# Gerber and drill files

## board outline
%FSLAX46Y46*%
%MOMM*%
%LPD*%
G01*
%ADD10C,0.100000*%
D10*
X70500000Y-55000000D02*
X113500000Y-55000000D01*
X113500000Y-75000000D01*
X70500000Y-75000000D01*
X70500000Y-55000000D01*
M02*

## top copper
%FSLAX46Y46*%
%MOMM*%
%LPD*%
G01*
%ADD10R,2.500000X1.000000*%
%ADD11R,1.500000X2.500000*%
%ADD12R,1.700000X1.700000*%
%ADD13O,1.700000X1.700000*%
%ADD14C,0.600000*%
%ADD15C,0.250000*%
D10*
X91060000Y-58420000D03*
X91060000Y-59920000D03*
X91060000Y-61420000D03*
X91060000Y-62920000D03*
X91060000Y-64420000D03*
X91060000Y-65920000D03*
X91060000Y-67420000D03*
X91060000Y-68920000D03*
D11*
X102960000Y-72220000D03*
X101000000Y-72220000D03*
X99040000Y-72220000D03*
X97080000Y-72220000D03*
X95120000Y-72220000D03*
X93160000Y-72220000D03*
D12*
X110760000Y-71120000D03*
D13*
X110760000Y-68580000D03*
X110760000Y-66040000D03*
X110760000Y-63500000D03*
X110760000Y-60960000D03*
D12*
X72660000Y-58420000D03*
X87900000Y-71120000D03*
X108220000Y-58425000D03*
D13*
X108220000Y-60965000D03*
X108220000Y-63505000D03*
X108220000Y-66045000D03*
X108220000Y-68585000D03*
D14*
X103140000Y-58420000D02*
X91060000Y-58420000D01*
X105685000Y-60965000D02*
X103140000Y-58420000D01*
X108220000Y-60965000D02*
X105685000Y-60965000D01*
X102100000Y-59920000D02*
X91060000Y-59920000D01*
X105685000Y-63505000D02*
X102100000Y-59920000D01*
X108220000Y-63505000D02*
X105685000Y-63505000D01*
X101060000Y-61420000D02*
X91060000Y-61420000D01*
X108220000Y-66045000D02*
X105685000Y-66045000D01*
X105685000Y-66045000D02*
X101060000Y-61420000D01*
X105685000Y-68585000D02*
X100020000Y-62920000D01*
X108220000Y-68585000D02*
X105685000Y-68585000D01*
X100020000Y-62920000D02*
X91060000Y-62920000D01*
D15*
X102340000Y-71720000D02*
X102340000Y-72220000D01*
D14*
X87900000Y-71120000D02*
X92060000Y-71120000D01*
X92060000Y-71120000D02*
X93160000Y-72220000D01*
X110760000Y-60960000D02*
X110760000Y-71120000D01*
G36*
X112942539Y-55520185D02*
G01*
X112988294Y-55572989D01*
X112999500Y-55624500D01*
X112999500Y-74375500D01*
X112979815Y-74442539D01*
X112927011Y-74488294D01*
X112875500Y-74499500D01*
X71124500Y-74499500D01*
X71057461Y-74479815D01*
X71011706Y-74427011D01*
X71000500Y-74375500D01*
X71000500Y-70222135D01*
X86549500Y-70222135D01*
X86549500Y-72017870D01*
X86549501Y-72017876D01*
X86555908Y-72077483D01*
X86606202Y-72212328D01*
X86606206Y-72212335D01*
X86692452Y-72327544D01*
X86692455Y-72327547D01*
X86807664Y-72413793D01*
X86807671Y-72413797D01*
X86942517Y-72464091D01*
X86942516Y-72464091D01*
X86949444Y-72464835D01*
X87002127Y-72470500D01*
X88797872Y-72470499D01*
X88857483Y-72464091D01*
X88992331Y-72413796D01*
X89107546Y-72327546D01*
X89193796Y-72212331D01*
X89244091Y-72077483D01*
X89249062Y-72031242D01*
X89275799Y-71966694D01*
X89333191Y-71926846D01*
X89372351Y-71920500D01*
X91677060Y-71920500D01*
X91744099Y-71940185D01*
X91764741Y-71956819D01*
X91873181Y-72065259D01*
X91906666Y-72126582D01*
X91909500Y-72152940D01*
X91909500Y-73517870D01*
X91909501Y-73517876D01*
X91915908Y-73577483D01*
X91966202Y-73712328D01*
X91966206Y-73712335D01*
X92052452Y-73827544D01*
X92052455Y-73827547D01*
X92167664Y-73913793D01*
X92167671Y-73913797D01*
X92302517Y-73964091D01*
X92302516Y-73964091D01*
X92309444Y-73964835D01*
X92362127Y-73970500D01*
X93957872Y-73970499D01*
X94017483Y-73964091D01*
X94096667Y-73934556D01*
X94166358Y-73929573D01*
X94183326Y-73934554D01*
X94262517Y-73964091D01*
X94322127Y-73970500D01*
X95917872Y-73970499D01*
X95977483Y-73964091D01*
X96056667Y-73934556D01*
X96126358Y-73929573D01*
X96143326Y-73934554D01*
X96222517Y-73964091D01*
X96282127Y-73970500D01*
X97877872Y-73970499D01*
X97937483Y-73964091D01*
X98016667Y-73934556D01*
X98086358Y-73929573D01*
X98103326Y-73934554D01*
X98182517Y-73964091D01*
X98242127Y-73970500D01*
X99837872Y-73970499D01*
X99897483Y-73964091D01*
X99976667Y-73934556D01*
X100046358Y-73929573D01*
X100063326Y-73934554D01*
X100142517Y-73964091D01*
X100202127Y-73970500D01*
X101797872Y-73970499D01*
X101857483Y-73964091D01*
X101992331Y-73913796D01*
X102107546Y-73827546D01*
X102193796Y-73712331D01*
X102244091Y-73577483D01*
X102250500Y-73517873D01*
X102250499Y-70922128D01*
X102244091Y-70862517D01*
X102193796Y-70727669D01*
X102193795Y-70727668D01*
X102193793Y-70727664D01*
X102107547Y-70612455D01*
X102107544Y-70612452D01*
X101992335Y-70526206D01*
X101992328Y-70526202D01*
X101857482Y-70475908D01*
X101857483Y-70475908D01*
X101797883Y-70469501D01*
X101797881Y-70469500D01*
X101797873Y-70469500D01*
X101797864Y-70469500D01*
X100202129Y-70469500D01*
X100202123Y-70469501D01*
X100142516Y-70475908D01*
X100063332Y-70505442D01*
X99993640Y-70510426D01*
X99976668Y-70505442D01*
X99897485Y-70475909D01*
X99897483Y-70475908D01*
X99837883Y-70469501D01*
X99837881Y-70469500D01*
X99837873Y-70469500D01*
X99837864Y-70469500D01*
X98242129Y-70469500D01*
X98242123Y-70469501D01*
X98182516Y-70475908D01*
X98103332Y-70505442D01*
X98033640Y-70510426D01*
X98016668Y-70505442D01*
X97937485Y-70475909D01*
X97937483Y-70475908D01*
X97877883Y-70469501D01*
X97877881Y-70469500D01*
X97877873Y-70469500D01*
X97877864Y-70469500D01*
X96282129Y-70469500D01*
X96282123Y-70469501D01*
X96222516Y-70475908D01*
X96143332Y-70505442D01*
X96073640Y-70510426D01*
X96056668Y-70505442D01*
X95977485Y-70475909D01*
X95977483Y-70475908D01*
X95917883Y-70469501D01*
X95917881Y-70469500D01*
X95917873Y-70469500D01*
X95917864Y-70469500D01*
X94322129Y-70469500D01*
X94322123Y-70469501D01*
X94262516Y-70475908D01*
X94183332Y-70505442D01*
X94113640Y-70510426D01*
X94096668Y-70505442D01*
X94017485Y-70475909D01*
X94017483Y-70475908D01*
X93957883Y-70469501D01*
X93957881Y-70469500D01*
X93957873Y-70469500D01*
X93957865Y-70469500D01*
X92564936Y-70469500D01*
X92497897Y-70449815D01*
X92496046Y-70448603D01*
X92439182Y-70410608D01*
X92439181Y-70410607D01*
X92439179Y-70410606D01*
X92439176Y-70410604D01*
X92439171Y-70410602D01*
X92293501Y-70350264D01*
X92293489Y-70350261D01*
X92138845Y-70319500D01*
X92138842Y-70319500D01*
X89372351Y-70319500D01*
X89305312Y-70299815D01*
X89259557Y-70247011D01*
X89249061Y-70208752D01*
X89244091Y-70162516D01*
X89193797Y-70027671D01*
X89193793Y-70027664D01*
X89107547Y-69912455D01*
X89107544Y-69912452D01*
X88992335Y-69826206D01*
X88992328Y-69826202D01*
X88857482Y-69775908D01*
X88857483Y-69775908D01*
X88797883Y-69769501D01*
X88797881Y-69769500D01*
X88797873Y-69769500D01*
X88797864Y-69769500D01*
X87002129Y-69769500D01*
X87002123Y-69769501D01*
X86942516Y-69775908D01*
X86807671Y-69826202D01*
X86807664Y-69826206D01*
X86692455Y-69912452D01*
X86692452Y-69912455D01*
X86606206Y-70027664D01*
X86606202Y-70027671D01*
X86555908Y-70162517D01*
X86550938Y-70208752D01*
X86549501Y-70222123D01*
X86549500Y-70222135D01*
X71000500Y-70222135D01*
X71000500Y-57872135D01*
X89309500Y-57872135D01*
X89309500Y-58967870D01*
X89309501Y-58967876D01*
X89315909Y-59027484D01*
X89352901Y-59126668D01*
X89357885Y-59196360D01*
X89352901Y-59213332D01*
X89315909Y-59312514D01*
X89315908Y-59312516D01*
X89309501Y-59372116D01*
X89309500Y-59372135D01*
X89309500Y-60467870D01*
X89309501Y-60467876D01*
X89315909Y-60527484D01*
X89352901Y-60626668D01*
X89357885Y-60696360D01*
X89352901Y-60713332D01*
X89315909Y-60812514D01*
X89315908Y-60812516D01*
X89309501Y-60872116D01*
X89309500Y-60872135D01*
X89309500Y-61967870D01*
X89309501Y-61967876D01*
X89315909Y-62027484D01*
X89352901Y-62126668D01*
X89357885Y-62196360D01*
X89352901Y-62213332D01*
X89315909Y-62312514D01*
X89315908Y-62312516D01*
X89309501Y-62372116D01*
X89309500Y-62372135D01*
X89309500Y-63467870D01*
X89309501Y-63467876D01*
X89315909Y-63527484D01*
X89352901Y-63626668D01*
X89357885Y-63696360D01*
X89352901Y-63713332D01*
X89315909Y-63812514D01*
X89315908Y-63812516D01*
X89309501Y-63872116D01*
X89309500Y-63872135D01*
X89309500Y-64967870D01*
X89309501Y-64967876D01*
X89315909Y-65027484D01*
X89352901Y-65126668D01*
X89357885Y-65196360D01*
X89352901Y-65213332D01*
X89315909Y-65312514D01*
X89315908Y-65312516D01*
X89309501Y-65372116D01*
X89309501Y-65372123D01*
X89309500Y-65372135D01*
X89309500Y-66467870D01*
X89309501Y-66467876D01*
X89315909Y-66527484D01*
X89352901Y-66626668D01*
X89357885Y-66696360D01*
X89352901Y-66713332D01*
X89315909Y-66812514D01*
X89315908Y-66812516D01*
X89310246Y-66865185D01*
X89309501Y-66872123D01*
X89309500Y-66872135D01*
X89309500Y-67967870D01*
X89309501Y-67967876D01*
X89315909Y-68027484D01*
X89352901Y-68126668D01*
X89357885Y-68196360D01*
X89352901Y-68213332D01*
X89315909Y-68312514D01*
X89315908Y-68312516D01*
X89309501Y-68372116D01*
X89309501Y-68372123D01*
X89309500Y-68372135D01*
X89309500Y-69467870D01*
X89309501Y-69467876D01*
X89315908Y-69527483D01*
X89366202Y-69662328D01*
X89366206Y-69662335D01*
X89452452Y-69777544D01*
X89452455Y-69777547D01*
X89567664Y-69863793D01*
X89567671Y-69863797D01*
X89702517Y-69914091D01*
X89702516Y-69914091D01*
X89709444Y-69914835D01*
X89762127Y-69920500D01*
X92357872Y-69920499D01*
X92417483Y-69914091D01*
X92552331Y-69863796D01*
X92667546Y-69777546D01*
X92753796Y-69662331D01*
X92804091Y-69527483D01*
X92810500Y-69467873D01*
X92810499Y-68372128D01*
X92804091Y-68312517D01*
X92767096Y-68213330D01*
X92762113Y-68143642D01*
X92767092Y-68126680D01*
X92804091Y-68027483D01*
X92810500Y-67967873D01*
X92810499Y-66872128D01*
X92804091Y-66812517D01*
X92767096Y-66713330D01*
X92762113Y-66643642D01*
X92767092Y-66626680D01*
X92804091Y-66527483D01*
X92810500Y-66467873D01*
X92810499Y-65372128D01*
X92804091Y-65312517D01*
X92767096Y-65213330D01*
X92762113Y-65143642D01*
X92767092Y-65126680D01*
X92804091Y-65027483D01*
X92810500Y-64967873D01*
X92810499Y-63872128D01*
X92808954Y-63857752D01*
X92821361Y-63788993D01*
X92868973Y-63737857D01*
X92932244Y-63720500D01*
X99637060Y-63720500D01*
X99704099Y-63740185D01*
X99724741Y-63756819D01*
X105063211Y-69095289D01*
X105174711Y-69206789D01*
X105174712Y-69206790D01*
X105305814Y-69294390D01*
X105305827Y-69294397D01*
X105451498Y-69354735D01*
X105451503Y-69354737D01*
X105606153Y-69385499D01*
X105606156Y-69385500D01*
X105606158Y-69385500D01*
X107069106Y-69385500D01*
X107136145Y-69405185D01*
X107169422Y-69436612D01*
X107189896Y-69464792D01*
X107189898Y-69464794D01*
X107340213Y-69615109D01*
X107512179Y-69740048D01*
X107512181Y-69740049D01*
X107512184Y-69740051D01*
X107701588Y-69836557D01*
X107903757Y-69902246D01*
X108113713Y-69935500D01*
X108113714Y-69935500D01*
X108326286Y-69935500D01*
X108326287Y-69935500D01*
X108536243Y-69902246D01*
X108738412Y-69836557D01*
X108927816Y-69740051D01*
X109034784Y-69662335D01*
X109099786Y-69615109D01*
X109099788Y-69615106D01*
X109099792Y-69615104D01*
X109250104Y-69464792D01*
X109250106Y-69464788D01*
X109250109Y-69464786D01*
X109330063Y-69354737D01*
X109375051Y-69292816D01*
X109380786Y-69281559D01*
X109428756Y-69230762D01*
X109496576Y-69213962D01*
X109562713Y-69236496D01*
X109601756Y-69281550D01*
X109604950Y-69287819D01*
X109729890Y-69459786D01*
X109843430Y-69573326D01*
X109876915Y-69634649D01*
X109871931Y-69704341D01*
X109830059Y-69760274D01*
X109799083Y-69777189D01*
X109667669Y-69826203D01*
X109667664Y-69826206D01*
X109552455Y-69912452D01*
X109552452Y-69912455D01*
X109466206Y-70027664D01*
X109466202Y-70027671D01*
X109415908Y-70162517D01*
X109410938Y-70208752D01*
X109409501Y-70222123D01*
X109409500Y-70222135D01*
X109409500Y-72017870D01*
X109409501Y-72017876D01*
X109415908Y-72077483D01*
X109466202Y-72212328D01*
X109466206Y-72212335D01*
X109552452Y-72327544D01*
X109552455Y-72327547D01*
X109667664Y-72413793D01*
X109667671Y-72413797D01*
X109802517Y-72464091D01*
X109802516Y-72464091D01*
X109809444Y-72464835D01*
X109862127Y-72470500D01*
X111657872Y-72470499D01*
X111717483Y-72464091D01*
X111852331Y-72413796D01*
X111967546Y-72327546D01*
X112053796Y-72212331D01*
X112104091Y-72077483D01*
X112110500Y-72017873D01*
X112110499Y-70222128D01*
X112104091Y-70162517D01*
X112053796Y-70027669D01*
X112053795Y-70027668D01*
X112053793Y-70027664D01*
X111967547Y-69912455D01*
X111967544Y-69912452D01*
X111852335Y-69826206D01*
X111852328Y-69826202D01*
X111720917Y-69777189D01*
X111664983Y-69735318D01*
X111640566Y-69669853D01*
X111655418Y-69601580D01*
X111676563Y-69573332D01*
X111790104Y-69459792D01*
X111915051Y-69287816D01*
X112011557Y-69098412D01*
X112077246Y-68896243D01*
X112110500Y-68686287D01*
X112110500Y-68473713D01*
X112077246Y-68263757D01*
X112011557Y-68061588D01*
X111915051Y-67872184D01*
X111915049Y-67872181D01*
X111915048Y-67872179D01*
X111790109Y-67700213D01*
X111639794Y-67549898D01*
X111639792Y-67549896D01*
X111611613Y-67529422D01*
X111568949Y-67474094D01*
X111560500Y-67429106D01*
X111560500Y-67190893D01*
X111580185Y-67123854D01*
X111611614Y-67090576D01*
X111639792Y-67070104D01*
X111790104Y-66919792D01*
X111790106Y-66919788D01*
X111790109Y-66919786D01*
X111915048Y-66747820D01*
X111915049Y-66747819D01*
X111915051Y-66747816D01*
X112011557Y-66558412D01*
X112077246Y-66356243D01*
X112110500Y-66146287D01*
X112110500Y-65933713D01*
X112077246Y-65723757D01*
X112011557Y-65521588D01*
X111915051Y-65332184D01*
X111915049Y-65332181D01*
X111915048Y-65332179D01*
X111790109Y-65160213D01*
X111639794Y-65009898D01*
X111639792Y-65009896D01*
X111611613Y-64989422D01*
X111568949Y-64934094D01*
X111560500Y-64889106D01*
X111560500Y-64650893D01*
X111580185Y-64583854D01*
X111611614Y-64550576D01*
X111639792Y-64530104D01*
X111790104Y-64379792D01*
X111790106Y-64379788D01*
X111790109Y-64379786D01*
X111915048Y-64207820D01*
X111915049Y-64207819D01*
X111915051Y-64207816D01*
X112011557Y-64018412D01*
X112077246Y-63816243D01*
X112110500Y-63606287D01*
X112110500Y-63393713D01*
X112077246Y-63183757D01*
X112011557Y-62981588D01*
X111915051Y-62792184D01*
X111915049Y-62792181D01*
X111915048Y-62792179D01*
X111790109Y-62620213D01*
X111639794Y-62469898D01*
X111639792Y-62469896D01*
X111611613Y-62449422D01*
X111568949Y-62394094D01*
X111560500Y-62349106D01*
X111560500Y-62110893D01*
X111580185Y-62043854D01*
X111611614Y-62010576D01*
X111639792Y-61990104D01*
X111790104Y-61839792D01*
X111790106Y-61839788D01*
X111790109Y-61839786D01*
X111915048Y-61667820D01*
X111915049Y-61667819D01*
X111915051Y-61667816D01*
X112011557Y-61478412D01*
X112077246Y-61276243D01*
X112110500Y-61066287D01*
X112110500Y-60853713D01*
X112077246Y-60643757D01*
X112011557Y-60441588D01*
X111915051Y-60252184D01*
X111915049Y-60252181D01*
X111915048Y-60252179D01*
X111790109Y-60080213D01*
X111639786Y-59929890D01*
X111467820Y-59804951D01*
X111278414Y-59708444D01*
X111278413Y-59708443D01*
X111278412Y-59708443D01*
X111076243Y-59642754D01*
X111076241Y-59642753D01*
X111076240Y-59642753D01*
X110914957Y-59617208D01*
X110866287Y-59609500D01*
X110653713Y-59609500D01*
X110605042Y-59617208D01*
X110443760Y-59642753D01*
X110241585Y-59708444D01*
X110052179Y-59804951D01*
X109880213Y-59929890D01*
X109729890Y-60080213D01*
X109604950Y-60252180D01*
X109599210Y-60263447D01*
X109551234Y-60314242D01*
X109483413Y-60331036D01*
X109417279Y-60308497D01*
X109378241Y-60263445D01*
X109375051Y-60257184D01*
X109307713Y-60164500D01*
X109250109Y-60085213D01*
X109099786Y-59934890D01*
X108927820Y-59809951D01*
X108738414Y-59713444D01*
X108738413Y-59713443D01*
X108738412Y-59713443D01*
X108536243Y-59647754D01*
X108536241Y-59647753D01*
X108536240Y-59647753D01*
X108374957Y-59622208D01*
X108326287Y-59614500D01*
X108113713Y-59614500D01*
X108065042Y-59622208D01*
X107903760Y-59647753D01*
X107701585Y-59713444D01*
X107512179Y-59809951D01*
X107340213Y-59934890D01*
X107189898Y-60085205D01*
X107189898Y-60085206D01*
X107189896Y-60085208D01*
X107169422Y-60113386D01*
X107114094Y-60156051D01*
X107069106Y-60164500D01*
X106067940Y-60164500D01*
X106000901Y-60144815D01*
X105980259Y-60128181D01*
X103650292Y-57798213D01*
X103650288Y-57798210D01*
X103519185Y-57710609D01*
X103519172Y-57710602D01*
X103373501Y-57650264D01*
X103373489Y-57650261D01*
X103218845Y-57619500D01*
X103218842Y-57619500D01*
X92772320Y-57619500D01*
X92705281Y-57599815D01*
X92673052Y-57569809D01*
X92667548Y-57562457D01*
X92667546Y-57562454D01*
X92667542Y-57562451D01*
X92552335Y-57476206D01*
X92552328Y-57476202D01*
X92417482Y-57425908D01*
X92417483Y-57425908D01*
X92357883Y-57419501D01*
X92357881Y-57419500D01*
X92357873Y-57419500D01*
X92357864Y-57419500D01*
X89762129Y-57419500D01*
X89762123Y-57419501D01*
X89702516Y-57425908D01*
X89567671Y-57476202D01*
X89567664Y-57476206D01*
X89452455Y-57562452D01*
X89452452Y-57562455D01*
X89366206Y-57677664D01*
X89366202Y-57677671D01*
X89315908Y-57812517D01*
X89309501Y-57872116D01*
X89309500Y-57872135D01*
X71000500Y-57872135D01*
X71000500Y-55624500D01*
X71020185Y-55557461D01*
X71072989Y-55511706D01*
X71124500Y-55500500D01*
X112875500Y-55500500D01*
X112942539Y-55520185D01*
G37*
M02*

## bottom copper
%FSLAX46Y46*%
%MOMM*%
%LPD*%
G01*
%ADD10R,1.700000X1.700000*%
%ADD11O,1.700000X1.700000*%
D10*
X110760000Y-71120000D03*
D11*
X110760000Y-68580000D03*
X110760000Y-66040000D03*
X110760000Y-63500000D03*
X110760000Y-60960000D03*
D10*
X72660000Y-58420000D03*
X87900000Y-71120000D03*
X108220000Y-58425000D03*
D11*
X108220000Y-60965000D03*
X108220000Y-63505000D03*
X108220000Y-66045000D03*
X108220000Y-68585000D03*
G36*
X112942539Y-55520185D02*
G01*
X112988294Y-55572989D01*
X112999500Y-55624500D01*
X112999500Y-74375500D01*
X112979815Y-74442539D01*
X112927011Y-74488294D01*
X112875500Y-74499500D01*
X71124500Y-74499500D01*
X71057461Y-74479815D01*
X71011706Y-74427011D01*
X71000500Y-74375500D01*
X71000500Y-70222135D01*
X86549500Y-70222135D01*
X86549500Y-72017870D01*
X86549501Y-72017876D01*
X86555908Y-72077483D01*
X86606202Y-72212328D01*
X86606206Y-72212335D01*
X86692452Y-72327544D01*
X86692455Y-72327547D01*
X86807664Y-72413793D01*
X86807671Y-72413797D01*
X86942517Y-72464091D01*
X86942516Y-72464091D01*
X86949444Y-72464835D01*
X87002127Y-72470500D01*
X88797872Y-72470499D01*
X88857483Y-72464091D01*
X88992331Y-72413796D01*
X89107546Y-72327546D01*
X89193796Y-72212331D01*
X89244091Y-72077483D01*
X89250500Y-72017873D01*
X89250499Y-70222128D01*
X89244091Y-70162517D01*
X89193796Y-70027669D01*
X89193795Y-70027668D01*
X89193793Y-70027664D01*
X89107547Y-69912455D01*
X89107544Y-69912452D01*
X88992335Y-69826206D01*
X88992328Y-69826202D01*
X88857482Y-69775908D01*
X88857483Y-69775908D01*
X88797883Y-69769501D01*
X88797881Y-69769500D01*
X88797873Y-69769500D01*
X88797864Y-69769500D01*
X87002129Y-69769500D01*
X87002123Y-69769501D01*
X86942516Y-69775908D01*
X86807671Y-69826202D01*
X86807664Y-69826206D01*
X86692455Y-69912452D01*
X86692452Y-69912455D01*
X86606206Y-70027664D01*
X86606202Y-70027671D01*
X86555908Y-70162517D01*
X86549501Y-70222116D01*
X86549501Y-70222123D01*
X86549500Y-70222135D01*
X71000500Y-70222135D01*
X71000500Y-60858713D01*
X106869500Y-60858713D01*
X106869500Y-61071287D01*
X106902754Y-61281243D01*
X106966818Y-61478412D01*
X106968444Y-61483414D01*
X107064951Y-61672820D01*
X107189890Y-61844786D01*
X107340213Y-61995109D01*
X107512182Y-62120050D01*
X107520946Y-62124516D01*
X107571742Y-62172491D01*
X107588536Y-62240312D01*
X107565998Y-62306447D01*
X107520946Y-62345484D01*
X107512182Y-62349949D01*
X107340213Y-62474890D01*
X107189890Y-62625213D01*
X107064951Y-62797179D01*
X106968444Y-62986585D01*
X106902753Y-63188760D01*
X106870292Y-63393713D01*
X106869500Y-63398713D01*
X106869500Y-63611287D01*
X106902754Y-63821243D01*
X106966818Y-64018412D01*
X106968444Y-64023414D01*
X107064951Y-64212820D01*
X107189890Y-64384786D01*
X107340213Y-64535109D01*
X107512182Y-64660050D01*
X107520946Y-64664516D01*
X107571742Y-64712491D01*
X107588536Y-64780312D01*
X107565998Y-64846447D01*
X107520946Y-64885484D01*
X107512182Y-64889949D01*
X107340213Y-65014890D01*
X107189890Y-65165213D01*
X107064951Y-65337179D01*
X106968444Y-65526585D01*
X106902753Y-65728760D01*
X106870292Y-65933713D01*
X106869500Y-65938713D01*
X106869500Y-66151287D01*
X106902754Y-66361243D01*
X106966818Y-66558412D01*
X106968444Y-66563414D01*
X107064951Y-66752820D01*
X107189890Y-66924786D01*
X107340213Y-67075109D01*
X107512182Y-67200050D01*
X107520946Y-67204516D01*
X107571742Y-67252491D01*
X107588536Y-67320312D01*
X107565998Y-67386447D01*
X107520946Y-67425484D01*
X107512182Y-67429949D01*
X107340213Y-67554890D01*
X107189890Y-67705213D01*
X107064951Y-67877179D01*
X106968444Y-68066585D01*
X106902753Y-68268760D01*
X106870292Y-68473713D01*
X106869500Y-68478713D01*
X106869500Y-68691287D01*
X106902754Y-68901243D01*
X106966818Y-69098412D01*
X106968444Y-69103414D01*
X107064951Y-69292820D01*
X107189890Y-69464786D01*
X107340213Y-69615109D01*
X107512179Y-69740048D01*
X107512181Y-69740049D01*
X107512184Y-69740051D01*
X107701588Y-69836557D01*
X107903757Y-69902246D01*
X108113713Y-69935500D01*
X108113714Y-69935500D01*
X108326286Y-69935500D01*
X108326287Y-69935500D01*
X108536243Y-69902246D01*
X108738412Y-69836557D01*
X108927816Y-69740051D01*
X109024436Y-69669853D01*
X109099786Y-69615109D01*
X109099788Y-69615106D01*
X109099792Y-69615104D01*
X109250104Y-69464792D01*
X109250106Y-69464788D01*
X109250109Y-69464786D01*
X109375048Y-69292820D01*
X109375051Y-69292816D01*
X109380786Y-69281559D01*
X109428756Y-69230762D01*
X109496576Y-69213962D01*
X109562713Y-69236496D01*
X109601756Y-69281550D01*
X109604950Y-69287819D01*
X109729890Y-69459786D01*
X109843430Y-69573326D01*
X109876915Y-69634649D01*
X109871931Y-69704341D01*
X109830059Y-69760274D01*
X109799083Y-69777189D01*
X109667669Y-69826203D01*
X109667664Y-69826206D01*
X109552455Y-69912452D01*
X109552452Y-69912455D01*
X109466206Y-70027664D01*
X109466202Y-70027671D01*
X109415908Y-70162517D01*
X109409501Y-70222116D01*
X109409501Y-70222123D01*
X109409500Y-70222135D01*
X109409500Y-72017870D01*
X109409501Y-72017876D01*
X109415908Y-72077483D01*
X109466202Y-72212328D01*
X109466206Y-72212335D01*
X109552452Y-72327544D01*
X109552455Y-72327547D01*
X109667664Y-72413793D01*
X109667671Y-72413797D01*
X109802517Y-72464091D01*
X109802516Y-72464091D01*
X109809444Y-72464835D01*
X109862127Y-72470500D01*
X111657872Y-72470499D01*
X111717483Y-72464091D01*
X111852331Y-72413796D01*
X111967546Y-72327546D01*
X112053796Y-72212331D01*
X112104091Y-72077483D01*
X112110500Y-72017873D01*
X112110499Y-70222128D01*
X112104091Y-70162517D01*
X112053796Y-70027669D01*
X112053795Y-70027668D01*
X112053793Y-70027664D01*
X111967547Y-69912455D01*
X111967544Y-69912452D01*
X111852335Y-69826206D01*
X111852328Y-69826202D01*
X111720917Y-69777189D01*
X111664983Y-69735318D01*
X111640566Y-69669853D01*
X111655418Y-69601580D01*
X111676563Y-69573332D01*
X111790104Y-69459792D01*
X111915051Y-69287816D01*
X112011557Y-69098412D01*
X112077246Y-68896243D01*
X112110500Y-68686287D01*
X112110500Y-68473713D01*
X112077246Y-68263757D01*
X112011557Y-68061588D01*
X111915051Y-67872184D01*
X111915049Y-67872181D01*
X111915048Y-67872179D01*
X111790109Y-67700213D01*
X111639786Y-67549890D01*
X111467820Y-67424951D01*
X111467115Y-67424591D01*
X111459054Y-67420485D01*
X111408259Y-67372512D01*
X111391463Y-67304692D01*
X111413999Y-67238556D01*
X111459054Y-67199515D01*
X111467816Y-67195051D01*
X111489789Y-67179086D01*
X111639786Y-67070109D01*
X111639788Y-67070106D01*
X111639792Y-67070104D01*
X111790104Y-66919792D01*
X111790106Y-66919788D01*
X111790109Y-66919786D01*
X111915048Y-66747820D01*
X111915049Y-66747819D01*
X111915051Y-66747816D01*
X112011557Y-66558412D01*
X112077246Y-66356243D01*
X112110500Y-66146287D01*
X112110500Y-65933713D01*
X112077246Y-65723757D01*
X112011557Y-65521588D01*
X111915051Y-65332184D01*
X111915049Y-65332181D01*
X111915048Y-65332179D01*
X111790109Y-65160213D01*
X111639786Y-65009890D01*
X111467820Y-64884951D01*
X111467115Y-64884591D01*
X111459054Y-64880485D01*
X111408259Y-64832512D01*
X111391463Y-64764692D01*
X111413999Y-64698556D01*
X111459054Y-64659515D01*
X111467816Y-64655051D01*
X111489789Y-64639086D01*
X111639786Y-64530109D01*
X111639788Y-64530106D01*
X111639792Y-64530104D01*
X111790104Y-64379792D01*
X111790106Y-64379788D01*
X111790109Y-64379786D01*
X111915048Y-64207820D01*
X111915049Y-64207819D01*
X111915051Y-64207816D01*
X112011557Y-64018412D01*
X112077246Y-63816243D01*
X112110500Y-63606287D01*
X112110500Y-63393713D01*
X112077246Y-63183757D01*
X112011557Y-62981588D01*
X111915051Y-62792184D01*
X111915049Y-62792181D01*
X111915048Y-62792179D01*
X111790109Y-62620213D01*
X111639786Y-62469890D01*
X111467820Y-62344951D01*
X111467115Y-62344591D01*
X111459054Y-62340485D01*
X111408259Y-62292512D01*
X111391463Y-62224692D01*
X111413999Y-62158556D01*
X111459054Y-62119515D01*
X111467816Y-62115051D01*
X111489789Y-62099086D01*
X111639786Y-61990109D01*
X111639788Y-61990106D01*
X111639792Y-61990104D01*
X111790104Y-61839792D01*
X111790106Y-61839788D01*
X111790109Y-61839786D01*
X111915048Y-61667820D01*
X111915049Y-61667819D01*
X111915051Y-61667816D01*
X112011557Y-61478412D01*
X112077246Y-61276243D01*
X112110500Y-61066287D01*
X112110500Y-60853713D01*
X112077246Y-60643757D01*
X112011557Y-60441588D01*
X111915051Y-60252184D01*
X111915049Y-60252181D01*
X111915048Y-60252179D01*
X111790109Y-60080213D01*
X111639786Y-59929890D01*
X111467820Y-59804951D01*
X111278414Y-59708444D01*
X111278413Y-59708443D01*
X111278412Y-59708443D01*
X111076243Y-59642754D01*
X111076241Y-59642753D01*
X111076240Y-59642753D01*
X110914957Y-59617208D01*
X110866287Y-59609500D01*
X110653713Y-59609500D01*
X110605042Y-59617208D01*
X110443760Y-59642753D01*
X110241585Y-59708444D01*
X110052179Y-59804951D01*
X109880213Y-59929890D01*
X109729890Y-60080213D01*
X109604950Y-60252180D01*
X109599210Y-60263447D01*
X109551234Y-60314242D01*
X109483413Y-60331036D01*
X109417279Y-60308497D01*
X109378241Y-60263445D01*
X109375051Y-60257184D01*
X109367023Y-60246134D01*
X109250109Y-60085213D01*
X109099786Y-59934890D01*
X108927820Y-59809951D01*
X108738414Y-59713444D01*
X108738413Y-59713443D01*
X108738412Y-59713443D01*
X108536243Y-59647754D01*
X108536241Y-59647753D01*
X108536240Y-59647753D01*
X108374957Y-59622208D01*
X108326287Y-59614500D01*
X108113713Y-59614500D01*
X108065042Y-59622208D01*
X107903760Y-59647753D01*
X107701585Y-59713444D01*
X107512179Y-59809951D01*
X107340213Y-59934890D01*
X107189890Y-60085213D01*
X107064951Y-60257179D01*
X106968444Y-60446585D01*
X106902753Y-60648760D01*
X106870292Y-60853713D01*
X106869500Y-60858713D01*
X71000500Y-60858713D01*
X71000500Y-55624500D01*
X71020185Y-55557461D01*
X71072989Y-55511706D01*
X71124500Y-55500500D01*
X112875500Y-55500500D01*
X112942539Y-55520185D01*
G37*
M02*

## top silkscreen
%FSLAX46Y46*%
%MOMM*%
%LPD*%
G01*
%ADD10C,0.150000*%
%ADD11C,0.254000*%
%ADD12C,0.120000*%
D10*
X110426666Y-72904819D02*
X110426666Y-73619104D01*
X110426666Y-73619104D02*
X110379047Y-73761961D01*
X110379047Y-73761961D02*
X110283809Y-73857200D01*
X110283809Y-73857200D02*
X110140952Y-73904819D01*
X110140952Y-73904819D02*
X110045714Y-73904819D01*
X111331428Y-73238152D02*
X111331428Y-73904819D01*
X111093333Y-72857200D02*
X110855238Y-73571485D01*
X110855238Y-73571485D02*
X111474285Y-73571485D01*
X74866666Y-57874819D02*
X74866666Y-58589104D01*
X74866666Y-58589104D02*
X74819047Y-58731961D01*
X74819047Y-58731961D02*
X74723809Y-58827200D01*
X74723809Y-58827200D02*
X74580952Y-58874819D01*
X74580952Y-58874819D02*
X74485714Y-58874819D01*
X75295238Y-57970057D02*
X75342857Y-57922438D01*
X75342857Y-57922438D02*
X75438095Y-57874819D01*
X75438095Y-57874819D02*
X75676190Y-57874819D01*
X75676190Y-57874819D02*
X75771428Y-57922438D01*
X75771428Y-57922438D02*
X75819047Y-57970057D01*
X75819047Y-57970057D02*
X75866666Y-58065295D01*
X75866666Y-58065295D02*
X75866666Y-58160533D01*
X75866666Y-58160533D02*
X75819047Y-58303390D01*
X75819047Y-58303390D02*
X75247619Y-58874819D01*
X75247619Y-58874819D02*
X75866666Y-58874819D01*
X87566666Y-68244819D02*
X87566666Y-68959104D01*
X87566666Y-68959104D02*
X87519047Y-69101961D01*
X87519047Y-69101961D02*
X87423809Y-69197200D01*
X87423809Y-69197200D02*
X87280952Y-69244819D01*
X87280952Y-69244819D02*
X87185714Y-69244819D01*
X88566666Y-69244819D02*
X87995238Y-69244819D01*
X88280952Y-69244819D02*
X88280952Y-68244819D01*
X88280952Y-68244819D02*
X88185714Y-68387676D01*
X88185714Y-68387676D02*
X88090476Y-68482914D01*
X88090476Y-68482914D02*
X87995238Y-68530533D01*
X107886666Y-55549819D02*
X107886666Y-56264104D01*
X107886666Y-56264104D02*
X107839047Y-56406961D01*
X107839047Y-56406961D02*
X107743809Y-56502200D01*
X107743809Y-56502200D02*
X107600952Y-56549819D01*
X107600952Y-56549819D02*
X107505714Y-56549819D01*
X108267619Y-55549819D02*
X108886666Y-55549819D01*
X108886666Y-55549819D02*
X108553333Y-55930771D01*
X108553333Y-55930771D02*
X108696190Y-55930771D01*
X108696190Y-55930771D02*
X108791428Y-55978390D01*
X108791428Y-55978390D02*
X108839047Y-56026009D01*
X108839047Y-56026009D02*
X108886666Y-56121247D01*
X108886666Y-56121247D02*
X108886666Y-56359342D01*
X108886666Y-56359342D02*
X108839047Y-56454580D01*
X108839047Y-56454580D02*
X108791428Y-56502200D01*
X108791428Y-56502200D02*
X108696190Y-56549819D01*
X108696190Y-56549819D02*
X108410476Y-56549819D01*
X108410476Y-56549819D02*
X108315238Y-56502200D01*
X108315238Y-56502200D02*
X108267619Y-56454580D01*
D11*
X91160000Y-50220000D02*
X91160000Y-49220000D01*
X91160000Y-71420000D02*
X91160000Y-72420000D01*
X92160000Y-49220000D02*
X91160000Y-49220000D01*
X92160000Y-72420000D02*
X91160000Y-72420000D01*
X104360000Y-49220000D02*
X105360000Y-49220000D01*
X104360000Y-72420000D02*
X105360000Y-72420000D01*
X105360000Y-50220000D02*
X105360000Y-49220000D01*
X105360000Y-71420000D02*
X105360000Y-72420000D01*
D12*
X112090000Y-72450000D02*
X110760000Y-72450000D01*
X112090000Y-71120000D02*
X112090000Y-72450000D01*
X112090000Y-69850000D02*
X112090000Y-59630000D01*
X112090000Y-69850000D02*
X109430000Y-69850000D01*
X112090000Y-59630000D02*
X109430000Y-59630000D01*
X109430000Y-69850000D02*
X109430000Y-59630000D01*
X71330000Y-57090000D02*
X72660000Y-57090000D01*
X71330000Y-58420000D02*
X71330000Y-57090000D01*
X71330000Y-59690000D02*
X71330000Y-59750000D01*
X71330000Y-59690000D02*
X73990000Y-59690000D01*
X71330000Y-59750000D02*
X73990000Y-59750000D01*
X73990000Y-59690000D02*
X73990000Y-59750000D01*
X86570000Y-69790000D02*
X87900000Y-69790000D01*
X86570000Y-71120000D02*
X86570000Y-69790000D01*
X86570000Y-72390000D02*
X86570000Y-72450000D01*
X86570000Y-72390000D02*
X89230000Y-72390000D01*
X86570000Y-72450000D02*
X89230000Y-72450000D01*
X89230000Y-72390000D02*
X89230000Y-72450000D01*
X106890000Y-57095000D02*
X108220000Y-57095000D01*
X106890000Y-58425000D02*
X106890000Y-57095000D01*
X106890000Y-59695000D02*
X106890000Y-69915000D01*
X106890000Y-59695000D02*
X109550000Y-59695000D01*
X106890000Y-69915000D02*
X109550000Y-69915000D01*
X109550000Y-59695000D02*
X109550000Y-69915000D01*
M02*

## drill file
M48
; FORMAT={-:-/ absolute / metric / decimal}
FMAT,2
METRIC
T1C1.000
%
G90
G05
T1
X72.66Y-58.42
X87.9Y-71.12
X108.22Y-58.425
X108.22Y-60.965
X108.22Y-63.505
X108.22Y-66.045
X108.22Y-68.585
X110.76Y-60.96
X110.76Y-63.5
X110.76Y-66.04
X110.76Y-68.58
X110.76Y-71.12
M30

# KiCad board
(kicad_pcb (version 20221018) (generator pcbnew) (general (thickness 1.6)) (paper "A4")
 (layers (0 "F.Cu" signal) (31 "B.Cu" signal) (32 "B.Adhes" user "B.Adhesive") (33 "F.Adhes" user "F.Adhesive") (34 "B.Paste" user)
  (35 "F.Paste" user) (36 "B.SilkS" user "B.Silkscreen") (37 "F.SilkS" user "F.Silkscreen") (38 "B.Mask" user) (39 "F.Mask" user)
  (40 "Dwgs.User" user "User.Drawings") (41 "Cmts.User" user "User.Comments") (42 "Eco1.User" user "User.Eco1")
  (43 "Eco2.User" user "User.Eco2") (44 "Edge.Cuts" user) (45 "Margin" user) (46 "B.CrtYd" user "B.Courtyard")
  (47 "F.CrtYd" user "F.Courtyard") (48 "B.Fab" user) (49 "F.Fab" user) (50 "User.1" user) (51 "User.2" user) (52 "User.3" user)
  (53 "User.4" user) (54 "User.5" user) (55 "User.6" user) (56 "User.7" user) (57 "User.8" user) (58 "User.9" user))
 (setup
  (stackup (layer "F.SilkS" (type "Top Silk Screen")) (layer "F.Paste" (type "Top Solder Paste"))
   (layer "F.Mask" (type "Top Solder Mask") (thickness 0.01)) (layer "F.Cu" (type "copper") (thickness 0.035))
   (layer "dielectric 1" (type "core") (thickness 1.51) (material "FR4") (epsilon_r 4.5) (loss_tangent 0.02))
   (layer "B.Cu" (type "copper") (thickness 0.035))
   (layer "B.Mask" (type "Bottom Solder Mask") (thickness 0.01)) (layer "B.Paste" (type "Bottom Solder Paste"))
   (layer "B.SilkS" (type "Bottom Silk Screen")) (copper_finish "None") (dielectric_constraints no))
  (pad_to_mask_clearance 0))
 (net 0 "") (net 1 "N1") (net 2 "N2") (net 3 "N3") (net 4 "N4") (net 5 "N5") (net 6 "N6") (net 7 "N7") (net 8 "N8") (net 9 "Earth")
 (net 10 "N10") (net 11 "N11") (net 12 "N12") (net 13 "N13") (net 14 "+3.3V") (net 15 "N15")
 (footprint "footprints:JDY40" (layer "F.Cu") (at 98.06 61.52)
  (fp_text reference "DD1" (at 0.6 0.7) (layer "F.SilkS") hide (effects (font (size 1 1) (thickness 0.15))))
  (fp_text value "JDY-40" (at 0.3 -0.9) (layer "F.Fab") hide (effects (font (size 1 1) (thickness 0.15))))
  (fp_line (start -6.9 -11.3) (end -6.9 -12.3) (stroke (width 0.254) (type solid)) (layer "F.SilkS"))
  (fp_line (start -6.9 9.9) (end -6.9 10.9) (stroke (width 0.254) (type solid)) (layer "F.SilkS"))
  (fp_line (start -5.9 -12.3) (end -6.9 -12.3) (stroke (width 0.254) (type solid)) (layer "F.SilkS"))
  (fp_line (start -5.9 10.9) (end -6.9 10.9) (stroke (width 0.254) (type solid)) (layer "F.SilkS"))
  (fp_line (start 6.3 -12.3) (end 7.3 -12.3) (stroke (width 0.254) (type solid)) (layer "F.SilkS"))
  (fp_line (start 6.3 10.9) (end 7.3 10.9) (stroke (width 0.254) (type solid)) (layer "F.SilkS"))
  (fp_line (start 7.3 -11.3) (end 7.3 -12.3) (stroke (width 0.254) (type solid)) (layer "F.SilkS"))
  (fp_line (start 7.3 9.9) (end 7.3 10.9) (stroke (width 0.254) (type solid)) (layer "F.SilkS"))
  (pad "1" smd rect (at -7 -3.1) (size 2.5 1) (layers "F.Cu" "F.Paste" "F.Mask") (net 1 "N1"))
  (pad "2" smd rect (at -7 -1.6) (size 2.5 1) (layers "F.Cu" "F.Paste" "F.Mask") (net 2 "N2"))
  (pad "3" smd rect (at -7 -0.1) (size 2.5 1) (layers "F.Cu" "F.Paste" "F.Mask") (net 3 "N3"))
  (pad "4" smd rect (at -7 1.4) (size 2.5 1) (layers "F.Cu" "F.Paste" "F.Mask") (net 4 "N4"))
  (pad "5" smd rect (at -7 2.9) (size 2.5 1) (layers "F.Cu" "F.Paste" "F.Mask") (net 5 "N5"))
  (pad "6" smd rect (at -7 4.4) (size 2.5 1) (layers "F.Cu" "F.Paste" "F.Mask") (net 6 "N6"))
  (pad "7" smd rect (at -7 5.9) (size 2.5 1) (layers "F.Cu" "F.Paste" "F.Mask") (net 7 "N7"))
  (pad "8" smd rect (at -7 7.4) (size 2.5 1) (layers "F.Cu" "F.Paste" "F.Mask") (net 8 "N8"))
  (pad "9" smd rect (at 4.9 10.7 90) (size 2.5 1.5) (layers "F.Cu" "F.Paste" "F.Mask") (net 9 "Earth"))
  (pad "10" smd rect (at 2.94 10.7 90) (size 2.5 1.5) (layers "F.Cu" "F.Paste" "F.Mask") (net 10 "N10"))
  (pad "11" smd rect (at 0.98 10.7 90) (size 2.5 1.5) (layers "F.Cu" "F.Paste" "F.Mask") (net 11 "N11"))
  (pad "12" smd rect (at -0.98 10.7 90) (size 2.5 1.5) (layers "F.Cu" "F.Paste" "F.Mask") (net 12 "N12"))
  (pad "13" smd rect (at -2.94 10.7 90) (size 2.5 1.5) (layers "F.Cu" "F.Paste" "F.Mask") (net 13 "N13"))
  (pad "14" smd rect (at -4.9 10.7 90) (size 2.5 1.5) (layers "F.Cu" "F.Paste" "F.Mask") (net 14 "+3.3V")))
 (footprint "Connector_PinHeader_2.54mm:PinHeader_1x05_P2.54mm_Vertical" (layer "F.Cu") (at 110.76 71.12 180)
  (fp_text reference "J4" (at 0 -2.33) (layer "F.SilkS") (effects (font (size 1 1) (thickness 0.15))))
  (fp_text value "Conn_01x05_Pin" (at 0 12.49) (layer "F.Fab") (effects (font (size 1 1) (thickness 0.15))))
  (fp_line (start -1.33 -1.33) (end 0 -1.33) (stroke (width 0.12) (type solid)) (layer "F.SilkS"))
  (fp_line (start -1.33 0) (end -1.33 -1.33) (stroke (width 0.12) (type solid)) (layer "F.SilkS"))
  (fp_line (start -1.33 1.27) (end -1.33 11.49) (stroke (width 0.12) (type solid)) (layer "F.SilkS"))
  (fp_line (start -1.33 1.27) (end 1.33 1.27) (stroke (width 0.12) (type solid)) (layer "F.SilkS"))
  (fp_line (start -1.33 11.49) (end 1.33 11.49) (stroke (width 0.12) (type solid)) (layer "F.SilkS"))
  (fp_line (start 1.33 1.27) (end 1.33 11.49) (stroke (width 0.12) (type solid)) (layer "F.SilkS"))
  (pad "1" thru_hole rect (at 0 0 180) (size 1.7 1.7) (drill 1) (layers "*.Cu" "*.Mask") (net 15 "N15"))
  (pad "2" thru_hole oval (at 0 2.54 180) (size 1.7 1.7) (drill 1) (layers "*.Cu" "*.Mask") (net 15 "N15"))
  (pad "3" thru_hole oval (at 0 5.08 180) (size 1.7 1.7) (drill 1) (layers "*.Cu" "*.Mask") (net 15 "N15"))
  (pad "4" thru_hole oval (at 0 7.62 180) (size 1.7 1.7) (drill 1) (layers "*.Cu" "*.Mask") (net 15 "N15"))
  (pad "5" thru_hole oval (at 0 10.16 180) (size 1.7 1.7) (drill 1) (layers "*.Cu" "*.Mask") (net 15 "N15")))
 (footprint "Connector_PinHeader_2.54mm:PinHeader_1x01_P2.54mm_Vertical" (layer "F.Cu") (at 72.66 58.42)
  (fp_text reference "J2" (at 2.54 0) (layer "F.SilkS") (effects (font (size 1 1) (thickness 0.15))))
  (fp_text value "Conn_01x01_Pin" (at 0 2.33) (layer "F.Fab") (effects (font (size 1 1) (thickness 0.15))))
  (fp_line (start -1.33 -1.33) (end 0 -1.33) (stroke (width 0.12) (type solid)) (layer "F.SilkS"))
  (fp_line (start -1.33 0) (end -1.33 -1.33) (stroke (width 0.12) (type solid)) (layer "F.SilkS"))
  (fp_line (start -1.33 1.27) (end -1.33 1.33) (stroke (width 0.12) (type solid)) (layer "F.SilkS"))
  (fp_line (start -1.33 1.27) (end 1.33 1.27) (stroke (width 0.12) (type solid)) (layer "F.SilkS"))
  (fp_line (start -1.33 1.33) (end 1.33 1.33) (stroke (width 0.12) (type solid)) (layer "F.SilkS"))
  (fp_line (start 1.33 1.27) (end 1.33 1.33) (stroke (width 0.12) (type solid)) (layer "F.SilkS"))
  (pad "1" thru_hole rect (at 0 0) (size 1.7 1.7) (drill 1) (layers "*.Cu" "*.Mask") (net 9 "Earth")))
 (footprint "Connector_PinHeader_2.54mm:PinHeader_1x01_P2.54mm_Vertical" (layer "F.Cu") (at 87.9 71.12)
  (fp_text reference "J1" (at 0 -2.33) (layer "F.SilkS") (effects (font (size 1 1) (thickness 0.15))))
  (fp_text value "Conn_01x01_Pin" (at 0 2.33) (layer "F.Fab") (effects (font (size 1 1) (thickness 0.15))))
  (fp_line (start -1.33 -1.33) (end 0 -1.33) (stroke (width 0.12) (type solid)) (layer "F.SilkS"))
  (fp_line (start -1.33 0) (end -1.33 -1.33) (stroke (width 0.12) (type solid)) (layer "F.SilkS"))
  (fp_line (start -1.33 1.27) (end -1.33 1.33) (stroke (width 0.12) (type solid)) (layer "F.SilkS"))
  (fp_line (start -1.33 1.27) (end 1.33 1.27) (stroke (width 0.12) (type solid)) (layer "F.SilkS"))
  (fp_line (start -1.33 1.33) (end 1.33 1.33) (stroke (width 0.12) (type solid)) (layer "F.SilkS"))
  (fp_line (start 1.33 1.27) (end 1.33 1.33) (stroke (width 0.12) (type solid)) (layer "F.SilkS"))
  (pad "1" thru_hole rect (at 0 0) (size 1.7 1.7) (drill 1) (layers "*.Cu" "*.Mask") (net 14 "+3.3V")))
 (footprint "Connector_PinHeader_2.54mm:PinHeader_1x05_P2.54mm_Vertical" (layer "F.Cu") (at 108.22 58.425)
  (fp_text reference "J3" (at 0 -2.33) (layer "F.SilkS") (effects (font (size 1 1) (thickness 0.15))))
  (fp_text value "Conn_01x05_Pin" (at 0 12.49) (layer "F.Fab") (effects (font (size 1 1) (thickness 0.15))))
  (fp_line (start -1.33 -1.33) (end 0 -1.33) (stroke (width 0.12) (type solid)) (layer "F.SilkS"))
  (fp_line (start -1.33 0) (end -1.33 -1.33) (stroke (width 0.12) (type solid)) (layer "F.SilkS"))
  (fp_line (start -1.33 1.27) (end -1.33 11.49) (stroke (width 0.12) (type solid)) (layer "F.SilkS"))
  (fp_line (start -1.33 1.27) (end 1.33 1.27) (stroke (width 0.12) (type solid)) (layer "F.SilkS"))
  (fp_line (start -1.33 11.49) (end 1.33 11.49) (stroke (width 0.12) (type solid)) (layer "F.SilkS"))
  (fp_line (start 1.33 1.27) (end 1.33 11.49) (stroke (width 0.12) (type solid)) (layer "F.SilkS"))
  (pad "1" thru_hole rect (at 0 0) (size 1.7 1.7) (drill 1) (layers "*.Cu" "*.Mask") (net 9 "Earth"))
  (pad "2" thru_hole oval (at 0 2.54) (size 1.7 1.7) (drill 1) (layers "*.Cu" "*.Mask") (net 1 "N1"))
  (pad "3" thru_hole oval (at 0 5.08) (size 1.7 1.7) (drill 1) (layers "*.Cu" "*.Mask") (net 2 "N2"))
  (pad "4" thru_hole oval (at 0 7.62) (size 1.7 1.7) (drill 1) (layers "*.Cu" "*.Mask") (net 3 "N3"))
  (pad "5" thru_hole oval (at 0 10.16) (size 1.7 1.7) (drill 1) (layers "*.Cu" "*.Mask") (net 4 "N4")))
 (gr_rect (start 70.5 55) (end 113.5 75) (stroke (width 0.1) (type default)) (fill none) (layer "Edge.Cuts"))
 (segment (start 103.14 58.42) (end 91.06 58.42) (width 0.6) (layer "F.Cu") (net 1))
 (segment (start 105.685 60.965) (end 103.14 58.42) (width 0.6) (layer "F.Cu") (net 1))
 (segment (start 108.22 60.965) (end 105.685 60.965) (width 0.6) (layer "F.Cu") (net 1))
 (segment (start 102.1 59.92) (end 91.06 59.92) (width 0.6) (layer "F.Cu") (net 2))
 (segment (start 105.685 63.505) (end 102.1 59.92) (width 0.6) (layer "F.Cu") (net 2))
 (segment (start 108.22 63.505) (end 105.685 63.505) (width 0.6) (layer "F.Cu") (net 2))
 (segment (start 101.06 61.42) (end 91.06 61.42) (width 0.6) (layer "F.Cu") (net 3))
 (segment (start 108.22 66.045) (end 105.685 66.045) (width 0.6) (layer "F.Cu") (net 3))
 (segment (start 105.685 66.045) (end 101.06 61.42) (width 0.6) (layer "F.Cu") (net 3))
 (segment (start 105.685 68.585) (end 100.02 62.92) (width 0.6) (layer "F.Cu") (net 4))
 (segment (start 108.22 68.585) (end 105.685 68.585) (width 0.6) (layer "F.Cu") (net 4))
 (segment (start 100.02 62.92) (end 91.06 62.92) (width 0.6) (layer "F.Cu") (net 4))
 (segment (start 102.34 71.72) (end 102.34 72.22) (width 0.25) (layer "F.Cu") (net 9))
 (segment (start 87.9 71.12) (end 92.06 71.12) (width 0.6) (layer "F.Cu") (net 14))
 (segment (start 92.06 71.12) (end 93.16 72.22) (width 0.6) (layer "F.Cu") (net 14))
 (segment (start 110.76 60.96) (end 110.76 71.12) (width 0.6) (layer "F.Cu") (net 15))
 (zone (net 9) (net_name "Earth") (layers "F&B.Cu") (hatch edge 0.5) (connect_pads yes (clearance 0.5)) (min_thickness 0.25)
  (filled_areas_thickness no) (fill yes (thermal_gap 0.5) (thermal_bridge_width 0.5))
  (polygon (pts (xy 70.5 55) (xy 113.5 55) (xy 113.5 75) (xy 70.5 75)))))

